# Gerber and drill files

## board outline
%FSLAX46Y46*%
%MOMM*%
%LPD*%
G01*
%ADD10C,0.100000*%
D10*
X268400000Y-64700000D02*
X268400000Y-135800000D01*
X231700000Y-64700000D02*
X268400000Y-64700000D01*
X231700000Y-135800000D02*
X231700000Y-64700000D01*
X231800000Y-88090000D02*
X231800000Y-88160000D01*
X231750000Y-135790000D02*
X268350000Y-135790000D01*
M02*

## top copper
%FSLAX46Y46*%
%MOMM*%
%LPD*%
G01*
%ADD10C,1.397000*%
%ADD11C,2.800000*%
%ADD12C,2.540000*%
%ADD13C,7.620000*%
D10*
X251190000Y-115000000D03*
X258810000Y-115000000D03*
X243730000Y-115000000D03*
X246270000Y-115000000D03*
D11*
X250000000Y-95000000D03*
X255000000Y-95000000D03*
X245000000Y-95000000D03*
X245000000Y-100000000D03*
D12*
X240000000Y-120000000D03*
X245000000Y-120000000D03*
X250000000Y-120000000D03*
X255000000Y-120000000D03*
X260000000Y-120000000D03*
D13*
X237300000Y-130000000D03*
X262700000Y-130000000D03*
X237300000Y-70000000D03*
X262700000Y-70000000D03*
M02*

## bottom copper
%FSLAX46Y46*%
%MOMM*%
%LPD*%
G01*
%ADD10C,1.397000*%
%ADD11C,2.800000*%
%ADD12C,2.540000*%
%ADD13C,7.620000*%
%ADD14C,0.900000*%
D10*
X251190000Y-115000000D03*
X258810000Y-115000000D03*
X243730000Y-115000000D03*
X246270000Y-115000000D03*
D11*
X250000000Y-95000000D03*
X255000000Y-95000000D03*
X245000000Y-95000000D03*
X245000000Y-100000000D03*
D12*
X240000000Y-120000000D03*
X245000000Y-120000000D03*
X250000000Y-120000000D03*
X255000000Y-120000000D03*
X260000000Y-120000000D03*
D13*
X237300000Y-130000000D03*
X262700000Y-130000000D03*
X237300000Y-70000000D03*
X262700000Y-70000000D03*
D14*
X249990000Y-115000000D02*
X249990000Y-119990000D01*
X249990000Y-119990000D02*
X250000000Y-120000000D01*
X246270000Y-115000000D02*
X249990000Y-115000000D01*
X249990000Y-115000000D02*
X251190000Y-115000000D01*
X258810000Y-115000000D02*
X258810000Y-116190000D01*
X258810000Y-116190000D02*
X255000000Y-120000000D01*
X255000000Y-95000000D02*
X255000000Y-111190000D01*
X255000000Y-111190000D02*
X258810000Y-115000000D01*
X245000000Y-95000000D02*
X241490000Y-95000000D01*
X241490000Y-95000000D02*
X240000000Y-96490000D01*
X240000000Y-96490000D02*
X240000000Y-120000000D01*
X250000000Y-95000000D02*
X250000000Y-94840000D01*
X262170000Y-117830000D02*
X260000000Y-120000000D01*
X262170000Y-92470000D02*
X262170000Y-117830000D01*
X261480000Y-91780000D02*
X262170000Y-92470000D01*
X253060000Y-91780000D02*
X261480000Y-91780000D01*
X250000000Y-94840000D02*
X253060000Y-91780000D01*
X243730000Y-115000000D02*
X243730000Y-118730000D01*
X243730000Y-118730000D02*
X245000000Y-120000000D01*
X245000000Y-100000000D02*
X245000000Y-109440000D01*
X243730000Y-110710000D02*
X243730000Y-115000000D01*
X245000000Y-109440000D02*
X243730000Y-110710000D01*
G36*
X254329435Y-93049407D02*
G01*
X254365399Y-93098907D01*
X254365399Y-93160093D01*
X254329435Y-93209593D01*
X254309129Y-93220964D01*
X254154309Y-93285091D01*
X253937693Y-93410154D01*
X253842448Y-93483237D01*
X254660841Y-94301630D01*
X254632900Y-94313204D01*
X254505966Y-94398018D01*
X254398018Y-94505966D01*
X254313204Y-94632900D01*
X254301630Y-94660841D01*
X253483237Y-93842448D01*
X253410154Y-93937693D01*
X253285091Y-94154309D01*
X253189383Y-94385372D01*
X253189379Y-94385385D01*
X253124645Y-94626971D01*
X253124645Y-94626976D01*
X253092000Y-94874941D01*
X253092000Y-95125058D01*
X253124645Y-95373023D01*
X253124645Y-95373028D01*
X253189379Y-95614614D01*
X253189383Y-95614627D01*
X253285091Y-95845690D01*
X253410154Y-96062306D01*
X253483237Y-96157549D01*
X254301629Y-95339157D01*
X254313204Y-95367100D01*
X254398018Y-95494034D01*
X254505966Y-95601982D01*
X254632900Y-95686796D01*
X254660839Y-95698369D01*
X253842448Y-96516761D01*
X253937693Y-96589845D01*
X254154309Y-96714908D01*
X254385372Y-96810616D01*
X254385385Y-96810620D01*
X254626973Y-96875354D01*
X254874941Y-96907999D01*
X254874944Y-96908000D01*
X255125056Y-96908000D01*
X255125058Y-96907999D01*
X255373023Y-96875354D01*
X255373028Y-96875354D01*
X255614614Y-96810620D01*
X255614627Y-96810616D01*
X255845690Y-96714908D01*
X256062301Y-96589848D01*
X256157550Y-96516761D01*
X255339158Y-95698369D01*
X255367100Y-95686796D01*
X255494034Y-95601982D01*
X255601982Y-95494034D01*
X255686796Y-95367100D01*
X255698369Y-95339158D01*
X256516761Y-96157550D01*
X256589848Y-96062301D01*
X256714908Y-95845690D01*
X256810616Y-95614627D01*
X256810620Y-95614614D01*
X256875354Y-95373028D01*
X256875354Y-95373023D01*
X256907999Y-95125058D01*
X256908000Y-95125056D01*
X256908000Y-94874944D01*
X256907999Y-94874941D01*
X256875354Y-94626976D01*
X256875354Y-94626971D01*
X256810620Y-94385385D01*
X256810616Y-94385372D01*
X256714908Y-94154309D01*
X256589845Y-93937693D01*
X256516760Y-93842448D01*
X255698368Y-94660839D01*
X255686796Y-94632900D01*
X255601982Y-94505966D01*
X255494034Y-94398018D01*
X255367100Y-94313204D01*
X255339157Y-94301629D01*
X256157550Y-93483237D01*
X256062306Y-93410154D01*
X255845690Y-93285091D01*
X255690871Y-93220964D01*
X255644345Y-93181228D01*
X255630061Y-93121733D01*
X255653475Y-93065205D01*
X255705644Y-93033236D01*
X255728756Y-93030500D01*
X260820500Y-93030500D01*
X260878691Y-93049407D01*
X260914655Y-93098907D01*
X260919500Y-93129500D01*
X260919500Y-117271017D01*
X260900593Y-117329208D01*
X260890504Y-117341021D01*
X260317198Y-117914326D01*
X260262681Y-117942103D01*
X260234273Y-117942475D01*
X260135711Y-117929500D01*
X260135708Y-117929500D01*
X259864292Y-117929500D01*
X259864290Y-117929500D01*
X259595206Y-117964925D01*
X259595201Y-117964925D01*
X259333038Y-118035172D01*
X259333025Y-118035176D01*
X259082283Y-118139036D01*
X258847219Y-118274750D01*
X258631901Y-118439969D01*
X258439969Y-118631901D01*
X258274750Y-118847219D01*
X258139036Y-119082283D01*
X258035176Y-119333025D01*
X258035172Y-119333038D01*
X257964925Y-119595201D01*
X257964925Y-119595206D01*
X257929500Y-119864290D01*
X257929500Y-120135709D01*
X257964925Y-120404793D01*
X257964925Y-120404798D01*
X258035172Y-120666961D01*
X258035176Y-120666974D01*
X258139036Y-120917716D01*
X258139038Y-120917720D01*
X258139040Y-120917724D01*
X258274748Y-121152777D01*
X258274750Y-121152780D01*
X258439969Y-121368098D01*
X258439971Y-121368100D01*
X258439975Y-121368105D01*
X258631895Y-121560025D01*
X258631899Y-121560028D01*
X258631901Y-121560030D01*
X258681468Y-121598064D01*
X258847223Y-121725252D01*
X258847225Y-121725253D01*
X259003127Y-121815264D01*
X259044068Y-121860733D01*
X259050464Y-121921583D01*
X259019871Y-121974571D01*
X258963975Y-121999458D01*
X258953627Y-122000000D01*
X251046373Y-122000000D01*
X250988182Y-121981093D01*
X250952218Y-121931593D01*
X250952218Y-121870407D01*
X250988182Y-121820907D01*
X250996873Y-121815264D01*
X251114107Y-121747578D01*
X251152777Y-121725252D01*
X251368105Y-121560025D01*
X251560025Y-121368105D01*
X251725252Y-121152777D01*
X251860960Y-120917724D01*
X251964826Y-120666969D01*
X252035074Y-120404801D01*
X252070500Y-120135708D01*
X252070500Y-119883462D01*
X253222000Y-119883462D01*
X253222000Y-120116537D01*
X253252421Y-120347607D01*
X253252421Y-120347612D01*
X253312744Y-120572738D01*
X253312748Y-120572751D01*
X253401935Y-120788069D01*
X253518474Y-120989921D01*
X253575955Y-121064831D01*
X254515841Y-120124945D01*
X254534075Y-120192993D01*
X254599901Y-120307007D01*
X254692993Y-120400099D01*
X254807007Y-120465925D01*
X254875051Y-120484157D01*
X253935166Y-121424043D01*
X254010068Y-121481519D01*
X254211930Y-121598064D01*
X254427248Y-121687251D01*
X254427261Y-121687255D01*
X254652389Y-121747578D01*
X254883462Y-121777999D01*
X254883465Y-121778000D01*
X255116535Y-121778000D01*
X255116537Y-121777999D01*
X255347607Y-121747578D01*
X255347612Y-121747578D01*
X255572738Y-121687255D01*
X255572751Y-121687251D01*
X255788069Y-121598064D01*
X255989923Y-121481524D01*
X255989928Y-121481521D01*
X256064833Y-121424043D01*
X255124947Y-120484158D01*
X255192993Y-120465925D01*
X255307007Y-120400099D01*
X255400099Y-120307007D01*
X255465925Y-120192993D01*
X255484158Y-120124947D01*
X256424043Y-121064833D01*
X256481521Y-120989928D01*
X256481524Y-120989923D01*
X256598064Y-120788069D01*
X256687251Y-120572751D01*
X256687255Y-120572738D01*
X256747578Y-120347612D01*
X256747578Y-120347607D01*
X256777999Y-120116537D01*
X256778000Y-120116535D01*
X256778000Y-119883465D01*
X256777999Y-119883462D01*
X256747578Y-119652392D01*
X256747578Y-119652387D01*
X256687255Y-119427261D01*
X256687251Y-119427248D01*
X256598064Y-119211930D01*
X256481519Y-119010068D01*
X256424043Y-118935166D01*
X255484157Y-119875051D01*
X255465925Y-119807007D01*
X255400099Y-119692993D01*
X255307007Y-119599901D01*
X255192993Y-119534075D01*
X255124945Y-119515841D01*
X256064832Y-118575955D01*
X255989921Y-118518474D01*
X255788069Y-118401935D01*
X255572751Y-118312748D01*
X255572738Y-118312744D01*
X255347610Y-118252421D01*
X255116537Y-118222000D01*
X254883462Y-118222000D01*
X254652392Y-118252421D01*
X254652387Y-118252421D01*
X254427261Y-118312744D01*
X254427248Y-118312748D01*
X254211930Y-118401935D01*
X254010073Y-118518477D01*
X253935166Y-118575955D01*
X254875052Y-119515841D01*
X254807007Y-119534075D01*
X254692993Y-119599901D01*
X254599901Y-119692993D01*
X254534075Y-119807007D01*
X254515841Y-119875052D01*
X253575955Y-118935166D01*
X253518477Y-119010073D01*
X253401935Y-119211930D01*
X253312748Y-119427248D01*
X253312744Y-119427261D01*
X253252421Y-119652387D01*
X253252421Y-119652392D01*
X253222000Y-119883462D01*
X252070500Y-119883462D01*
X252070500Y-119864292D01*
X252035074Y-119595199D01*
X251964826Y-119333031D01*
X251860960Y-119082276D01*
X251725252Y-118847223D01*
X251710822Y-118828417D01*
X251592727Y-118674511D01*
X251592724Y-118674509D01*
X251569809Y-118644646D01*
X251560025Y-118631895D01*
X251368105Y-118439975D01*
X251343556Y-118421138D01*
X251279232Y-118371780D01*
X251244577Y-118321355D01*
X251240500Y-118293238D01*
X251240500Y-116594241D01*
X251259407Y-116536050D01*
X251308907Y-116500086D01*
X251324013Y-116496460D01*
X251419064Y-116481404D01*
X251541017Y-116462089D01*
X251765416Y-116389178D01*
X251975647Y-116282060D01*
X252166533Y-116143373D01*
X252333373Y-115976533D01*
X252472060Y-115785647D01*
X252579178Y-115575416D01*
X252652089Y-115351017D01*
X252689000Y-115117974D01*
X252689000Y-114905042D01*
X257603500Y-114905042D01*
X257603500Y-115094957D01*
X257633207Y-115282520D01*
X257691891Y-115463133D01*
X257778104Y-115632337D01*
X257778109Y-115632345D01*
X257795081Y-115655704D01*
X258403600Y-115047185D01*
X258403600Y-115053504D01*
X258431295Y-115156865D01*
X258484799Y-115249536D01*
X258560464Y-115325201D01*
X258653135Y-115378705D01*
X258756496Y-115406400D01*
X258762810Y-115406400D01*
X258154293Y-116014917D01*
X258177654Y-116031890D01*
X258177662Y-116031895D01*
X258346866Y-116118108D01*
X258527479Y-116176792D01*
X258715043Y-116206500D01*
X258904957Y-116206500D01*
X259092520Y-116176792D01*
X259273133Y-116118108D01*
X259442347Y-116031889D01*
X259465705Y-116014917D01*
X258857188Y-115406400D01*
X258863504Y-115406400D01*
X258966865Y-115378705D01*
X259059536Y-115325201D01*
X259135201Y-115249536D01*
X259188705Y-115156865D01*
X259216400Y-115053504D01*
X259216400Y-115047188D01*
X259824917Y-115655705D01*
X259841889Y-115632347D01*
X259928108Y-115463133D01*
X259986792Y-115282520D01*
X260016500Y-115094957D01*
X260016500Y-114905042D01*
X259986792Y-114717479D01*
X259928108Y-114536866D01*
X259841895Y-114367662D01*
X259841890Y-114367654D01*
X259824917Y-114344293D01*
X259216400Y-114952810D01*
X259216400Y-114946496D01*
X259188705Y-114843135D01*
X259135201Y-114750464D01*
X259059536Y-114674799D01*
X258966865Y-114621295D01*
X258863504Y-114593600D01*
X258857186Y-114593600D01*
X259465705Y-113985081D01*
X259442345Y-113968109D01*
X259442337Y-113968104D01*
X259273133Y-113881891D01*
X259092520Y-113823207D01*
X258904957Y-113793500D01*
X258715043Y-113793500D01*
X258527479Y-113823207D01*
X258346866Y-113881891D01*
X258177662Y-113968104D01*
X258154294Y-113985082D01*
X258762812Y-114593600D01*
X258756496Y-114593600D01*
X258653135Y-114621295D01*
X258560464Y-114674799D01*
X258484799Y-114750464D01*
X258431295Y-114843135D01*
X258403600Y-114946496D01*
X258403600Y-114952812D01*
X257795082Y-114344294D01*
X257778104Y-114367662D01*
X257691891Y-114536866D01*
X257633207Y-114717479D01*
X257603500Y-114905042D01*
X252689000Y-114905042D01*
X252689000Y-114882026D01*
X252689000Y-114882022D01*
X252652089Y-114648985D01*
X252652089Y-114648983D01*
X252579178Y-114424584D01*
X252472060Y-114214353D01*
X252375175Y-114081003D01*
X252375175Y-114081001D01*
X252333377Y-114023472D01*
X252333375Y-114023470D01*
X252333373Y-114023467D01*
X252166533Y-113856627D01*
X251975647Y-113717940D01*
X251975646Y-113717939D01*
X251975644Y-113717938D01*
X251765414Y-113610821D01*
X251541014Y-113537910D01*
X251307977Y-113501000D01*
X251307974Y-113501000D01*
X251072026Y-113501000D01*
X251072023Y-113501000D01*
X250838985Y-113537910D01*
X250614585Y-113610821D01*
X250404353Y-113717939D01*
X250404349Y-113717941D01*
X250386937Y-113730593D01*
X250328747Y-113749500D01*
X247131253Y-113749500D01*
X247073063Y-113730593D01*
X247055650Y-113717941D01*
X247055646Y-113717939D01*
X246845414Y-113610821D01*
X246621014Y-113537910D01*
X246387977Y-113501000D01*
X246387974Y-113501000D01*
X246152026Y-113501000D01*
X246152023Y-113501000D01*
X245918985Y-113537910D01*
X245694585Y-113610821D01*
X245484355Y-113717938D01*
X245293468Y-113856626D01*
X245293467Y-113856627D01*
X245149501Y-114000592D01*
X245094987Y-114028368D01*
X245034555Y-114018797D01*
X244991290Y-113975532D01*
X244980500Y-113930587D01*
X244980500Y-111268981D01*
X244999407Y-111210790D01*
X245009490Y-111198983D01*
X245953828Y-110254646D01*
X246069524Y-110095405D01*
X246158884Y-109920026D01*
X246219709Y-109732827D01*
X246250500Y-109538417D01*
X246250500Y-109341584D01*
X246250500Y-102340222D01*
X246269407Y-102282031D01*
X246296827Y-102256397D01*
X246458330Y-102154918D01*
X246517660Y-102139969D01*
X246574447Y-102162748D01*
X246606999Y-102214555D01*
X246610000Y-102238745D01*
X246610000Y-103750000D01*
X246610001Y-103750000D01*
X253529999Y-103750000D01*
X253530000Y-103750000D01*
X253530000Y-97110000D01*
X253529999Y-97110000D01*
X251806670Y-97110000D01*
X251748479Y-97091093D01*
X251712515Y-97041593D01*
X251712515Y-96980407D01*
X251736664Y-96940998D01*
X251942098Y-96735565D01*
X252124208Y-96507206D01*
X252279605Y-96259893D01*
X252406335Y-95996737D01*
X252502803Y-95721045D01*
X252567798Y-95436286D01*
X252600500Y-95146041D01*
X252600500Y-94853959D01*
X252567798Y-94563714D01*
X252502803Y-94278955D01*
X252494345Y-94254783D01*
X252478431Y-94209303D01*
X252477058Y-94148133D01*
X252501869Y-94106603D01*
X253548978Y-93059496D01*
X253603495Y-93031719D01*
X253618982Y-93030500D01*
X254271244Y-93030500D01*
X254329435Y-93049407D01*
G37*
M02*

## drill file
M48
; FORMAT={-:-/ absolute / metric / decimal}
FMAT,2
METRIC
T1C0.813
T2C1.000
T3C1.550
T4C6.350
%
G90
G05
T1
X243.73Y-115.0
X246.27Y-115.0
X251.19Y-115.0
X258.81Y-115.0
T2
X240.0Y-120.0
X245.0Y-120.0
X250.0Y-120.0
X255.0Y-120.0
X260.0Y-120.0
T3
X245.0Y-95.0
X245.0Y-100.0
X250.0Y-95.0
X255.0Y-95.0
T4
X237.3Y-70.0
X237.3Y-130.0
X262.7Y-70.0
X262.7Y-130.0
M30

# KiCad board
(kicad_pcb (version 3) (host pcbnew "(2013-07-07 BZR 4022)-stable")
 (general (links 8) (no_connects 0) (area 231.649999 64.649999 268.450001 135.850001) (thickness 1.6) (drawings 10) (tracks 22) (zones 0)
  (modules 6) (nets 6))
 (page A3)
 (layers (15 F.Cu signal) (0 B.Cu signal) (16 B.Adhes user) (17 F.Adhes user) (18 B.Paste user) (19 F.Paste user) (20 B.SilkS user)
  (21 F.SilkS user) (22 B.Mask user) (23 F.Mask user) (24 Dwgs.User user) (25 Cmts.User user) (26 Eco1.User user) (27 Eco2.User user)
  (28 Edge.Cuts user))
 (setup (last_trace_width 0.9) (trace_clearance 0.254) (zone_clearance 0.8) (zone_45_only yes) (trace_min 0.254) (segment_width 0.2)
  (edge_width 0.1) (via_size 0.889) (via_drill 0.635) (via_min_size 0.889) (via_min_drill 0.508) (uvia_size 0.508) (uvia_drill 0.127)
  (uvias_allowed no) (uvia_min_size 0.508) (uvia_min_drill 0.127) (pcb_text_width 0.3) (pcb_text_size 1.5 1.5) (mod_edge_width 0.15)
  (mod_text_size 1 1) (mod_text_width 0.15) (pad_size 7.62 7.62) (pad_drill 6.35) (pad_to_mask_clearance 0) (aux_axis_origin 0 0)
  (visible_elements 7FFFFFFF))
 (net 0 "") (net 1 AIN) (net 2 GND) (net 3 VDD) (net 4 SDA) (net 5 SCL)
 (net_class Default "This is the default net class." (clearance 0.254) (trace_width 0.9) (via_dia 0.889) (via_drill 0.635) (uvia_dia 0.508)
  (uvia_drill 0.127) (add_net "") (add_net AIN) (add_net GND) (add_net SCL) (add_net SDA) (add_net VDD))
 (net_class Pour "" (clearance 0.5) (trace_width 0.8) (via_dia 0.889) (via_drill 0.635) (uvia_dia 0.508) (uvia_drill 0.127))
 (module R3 (layer F.Cu) (at 255 115) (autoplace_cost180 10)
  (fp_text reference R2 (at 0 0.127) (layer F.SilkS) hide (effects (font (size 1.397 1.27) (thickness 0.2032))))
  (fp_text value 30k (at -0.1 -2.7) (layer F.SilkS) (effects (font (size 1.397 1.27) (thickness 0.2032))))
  (pad 1 thru_hole circle (at -3.81 0) (size 1.397 1.397) (drill 0.8128) (layers *.Cu *.Mask F.SilkS) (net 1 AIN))
  (pad 2 thru_hole circle (at 3.81 0) (size 1.397 1.397) (drill 0.8128) (layers *.Cu *.Mask F.SilkS) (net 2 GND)))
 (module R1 (layer F.Cu) (at 245 115) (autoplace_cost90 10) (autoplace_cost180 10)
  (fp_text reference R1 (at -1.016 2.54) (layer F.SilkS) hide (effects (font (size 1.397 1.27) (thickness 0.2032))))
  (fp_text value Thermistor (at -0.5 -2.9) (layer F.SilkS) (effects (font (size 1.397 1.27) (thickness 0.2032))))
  (pad 1 thru_hole circle (at -1.27 0) (size 1.397 1.397) (drill 0.8128) (layers *.Cu *.Mask F.SilkS) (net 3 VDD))
  (pad 2 thru_hole circle (at 1.27 0) (size 1.397 1.397) (drill 0.8128) (layers *.Cu *.Mask F.SilkS) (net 1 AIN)))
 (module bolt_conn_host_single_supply (layer F.Cu) (at 250 100) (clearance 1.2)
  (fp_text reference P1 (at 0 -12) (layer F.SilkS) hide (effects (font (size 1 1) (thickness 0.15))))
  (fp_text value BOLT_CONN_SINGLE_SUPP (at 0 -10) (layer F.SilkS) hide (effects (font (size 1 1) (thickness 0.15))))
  (pad 4 thru_hole circle (at 0 -5) (size 2.8 2.8) (drill 1.55) (layers *.Cu F.SilkS F.Mask) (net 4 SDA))
  (pad 2 thru_hole circle (at 5 -5) (size 2.8 2.8) (drill 1.55) (layers *.Cu F.SilkS F.Mask) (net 2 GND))
  (pad 3 thru_hole circle (at -5 -5) (size 2.8 2.8) (drill 1.55) (layers *.Cu F.SilkS F.Mask) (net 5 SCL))
  (pad 1 thru_hole circle (at -5 0) (size 2.8 2.8) (drill 1.55) (layers *.Cu F.SilkS F.Mask) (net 3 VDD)))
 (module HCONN (layer F.Cu) (at 250 120)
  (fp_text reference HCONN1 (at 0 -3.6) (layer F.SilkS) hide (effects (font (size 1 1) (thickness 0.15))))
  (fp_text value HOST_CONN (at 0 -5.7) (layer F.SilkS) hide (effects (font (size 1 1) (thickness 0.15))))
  (pad 3 thru_hole circle (at -10 0) (size 2.54 2.54) (drill 1) (layers *.Cu *.Mask F.SilkS) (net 5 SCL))
  (pad 1 thru_hole circle (at -5 0) (size 2.54 2.54) (drill 1) (layers *.Cu *.Mask F.SilkS) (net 3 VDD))
  (pad 5 thru_hole circle (at 0 0) (size 2.54 2.54) (drill 1) (layers *.Cu *.Mask F.SilkS) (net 1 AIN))
  (pad 2 thru_hole circle (at 5 0) (size 2.54 2.54) (drill 1) (layers *.Cu *.Mask F.SilkS) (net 2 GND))
  (pad 4 thru_hole circle (at 10 0) (size 2.54 2.54) (drill 1) (layers *.Cu *.Mask F.SilkS) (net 4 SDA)))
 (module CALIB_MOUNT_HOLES (layer F.Cu) (at 250 130) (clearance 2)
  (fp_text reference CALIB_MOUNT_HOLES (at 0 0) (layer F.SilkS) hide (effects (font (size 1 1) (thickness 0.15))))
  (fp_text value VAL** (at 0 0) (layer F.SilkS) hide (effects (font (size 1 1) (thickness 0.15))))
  (pad "" np_thru_hole circle (at -12.7 0) (size 7.62 7.62) (drill 6.35) (layers *.Cu *.Mask F.SilkS) (clearance 3))
  (pad "" np_thru_hole circle (at 12.7 0) (size 7.62 7.62) (drill 6.35) (layers *.Cu *.Mask F.SilkS) (solder_paste_margin -7.62)
   (clearance 3)))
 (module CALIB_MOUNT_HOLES (layer F.Cu) (at 250 70)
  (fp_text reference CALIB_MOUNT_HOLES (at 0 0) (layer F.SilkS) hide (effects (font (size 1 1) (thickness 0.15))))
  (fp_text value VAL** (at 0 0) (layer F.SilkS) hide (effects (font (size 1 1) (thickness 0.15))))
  (pad "" np_thru_hole circle (at -12.7 0) (size 7.62 7.62) (drill 6.35) (layers *.Cu *.Mask F.SilkS) (clearance 1.27))
  (pad "" np_thru_hole circle (at 12.7 0) (size 7.62 7.62) (drill 6.35) (layers *.Cu *.Mask F.SilkS) (solder_paste_margin -7.62)
   (clearance 1.27)))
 (gr_line (start 268.4 64.7) (end 268.4 135.8) (angle 90) (layer Edge.Cuts) (width 0.1))
 (gr_line (start 231.7 64.7) (end 268.4 64.7) (angle 90) (layer Edge.Cuts) (width 0.1))
 (gr_line (start 231.7 135.8) (end 231.7 64.7) (angle 90) (layer Edge.Cuts) (width 0.1))
 (gr_line (start 231.8 88.09) (end 231.8 88.16) (angle 90) (layer Edge.Cuts) (width 0.1))
 (gr_line (start 231.75 135.79) (end 268.35 135.79) (angle 90) (layer Edge.Cuts) (width 0.1))
 (segment (start 249.99 115) (end 249.99 119.99) (width 0.9) (layer B.Cu) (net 1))
 (segment (start 249.99 119.99) (end 250 120) (width 0.9) (layer B.Cu) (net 1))
 (segment (start 246.27 115) (end 249.99 115) (width 0.9) (layer B.Cu) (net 1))
 (segment (start 249.99 115) (end 251.19 115) (width 0.9) (layer B.Cu) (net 1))
 (segment (start 258.81 115) (end 258.81 116.19) (width 0.9) (layer B.Cu) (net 2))
 (segment (start 258.81 116.19) (end 255 120) (width 0.9) (layer B.Cu) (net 2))
 (segment (start 255 95) (end 255 111.19) (width 0.9) (layer B.Cu) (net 2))
 (segment (start 255 111.19) (end 258.81 115) (width 0.9) (layer B.Cu) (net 2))
 (segment (start 245 95) (end 241.49 95) (width 0.9) (layer B.Cu) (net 5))
 (segment (start 241.49 95) (end 240 96.49) (width 0.9) (layer B.Cu) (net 5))
 (segment (start 240 96.49) (end 240 120) (width 0.9) (layer B.Cu) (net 5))
 (segment (start 250 95) (end 250 94.84) (width 0.9) (layer B.Cu) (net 4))
 (segment (start 262.17 117.83) (end 260 120) (width 0.9) (layer B.Cu) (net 4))
 (segment (start 262.17 92.47) (end 262.17 117.83) (width 0.9) (layer B.Cu) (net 4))
 (segment (start 261.48 91.78) (end 262.17 92.47) (width 0.9) (layer B.Cu) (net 4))
 (segment (start 253.06 91.78) (end 261.48 91.78) (width 0.9) (layer B.Cu) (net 4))
 (segment (start 250 94.84) (end 253.06 91.78) (width 0.9) (layer B.Cu) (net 4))
 (segment (start 243.73 115) (end 243.73 118.73) (width 0.9) (layer B.Cu) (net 3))
 (segment (start 243.73 118.73) (end 245 120) (width 0.9) (layer B.Cu) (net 3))
 (segment (start 245 100) (end 245 109.44) (width 0.9) (layer B.Cu) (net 3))
 (segment (start 243.73 110.71) (end 243.73 115) (width 0.9) (layer B.Cu) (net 3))
 (segment (start 245 109.44) (end 243.73 110.71) (width 0.9) (layer B.Cu) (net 3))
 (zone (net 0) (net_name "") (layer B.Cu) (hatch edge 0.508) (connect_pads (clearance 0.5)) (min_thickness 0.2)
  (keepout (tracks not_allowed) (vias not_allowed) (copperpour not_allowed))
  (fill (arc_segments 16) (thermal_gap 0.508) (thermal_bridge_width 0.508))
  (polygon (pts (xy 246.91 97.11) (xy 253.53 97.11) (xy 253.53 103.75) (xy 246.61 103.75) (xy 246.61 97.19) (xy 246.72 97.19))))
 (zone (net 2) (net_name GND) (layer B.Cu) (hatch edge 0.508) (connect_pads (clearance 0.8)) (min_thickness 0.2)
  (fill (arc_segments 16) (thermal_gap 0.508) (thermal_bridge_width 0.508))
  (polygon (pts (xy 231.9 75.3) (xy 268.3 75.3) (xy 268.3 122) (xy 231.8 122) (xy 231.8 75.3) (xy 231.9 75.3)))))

